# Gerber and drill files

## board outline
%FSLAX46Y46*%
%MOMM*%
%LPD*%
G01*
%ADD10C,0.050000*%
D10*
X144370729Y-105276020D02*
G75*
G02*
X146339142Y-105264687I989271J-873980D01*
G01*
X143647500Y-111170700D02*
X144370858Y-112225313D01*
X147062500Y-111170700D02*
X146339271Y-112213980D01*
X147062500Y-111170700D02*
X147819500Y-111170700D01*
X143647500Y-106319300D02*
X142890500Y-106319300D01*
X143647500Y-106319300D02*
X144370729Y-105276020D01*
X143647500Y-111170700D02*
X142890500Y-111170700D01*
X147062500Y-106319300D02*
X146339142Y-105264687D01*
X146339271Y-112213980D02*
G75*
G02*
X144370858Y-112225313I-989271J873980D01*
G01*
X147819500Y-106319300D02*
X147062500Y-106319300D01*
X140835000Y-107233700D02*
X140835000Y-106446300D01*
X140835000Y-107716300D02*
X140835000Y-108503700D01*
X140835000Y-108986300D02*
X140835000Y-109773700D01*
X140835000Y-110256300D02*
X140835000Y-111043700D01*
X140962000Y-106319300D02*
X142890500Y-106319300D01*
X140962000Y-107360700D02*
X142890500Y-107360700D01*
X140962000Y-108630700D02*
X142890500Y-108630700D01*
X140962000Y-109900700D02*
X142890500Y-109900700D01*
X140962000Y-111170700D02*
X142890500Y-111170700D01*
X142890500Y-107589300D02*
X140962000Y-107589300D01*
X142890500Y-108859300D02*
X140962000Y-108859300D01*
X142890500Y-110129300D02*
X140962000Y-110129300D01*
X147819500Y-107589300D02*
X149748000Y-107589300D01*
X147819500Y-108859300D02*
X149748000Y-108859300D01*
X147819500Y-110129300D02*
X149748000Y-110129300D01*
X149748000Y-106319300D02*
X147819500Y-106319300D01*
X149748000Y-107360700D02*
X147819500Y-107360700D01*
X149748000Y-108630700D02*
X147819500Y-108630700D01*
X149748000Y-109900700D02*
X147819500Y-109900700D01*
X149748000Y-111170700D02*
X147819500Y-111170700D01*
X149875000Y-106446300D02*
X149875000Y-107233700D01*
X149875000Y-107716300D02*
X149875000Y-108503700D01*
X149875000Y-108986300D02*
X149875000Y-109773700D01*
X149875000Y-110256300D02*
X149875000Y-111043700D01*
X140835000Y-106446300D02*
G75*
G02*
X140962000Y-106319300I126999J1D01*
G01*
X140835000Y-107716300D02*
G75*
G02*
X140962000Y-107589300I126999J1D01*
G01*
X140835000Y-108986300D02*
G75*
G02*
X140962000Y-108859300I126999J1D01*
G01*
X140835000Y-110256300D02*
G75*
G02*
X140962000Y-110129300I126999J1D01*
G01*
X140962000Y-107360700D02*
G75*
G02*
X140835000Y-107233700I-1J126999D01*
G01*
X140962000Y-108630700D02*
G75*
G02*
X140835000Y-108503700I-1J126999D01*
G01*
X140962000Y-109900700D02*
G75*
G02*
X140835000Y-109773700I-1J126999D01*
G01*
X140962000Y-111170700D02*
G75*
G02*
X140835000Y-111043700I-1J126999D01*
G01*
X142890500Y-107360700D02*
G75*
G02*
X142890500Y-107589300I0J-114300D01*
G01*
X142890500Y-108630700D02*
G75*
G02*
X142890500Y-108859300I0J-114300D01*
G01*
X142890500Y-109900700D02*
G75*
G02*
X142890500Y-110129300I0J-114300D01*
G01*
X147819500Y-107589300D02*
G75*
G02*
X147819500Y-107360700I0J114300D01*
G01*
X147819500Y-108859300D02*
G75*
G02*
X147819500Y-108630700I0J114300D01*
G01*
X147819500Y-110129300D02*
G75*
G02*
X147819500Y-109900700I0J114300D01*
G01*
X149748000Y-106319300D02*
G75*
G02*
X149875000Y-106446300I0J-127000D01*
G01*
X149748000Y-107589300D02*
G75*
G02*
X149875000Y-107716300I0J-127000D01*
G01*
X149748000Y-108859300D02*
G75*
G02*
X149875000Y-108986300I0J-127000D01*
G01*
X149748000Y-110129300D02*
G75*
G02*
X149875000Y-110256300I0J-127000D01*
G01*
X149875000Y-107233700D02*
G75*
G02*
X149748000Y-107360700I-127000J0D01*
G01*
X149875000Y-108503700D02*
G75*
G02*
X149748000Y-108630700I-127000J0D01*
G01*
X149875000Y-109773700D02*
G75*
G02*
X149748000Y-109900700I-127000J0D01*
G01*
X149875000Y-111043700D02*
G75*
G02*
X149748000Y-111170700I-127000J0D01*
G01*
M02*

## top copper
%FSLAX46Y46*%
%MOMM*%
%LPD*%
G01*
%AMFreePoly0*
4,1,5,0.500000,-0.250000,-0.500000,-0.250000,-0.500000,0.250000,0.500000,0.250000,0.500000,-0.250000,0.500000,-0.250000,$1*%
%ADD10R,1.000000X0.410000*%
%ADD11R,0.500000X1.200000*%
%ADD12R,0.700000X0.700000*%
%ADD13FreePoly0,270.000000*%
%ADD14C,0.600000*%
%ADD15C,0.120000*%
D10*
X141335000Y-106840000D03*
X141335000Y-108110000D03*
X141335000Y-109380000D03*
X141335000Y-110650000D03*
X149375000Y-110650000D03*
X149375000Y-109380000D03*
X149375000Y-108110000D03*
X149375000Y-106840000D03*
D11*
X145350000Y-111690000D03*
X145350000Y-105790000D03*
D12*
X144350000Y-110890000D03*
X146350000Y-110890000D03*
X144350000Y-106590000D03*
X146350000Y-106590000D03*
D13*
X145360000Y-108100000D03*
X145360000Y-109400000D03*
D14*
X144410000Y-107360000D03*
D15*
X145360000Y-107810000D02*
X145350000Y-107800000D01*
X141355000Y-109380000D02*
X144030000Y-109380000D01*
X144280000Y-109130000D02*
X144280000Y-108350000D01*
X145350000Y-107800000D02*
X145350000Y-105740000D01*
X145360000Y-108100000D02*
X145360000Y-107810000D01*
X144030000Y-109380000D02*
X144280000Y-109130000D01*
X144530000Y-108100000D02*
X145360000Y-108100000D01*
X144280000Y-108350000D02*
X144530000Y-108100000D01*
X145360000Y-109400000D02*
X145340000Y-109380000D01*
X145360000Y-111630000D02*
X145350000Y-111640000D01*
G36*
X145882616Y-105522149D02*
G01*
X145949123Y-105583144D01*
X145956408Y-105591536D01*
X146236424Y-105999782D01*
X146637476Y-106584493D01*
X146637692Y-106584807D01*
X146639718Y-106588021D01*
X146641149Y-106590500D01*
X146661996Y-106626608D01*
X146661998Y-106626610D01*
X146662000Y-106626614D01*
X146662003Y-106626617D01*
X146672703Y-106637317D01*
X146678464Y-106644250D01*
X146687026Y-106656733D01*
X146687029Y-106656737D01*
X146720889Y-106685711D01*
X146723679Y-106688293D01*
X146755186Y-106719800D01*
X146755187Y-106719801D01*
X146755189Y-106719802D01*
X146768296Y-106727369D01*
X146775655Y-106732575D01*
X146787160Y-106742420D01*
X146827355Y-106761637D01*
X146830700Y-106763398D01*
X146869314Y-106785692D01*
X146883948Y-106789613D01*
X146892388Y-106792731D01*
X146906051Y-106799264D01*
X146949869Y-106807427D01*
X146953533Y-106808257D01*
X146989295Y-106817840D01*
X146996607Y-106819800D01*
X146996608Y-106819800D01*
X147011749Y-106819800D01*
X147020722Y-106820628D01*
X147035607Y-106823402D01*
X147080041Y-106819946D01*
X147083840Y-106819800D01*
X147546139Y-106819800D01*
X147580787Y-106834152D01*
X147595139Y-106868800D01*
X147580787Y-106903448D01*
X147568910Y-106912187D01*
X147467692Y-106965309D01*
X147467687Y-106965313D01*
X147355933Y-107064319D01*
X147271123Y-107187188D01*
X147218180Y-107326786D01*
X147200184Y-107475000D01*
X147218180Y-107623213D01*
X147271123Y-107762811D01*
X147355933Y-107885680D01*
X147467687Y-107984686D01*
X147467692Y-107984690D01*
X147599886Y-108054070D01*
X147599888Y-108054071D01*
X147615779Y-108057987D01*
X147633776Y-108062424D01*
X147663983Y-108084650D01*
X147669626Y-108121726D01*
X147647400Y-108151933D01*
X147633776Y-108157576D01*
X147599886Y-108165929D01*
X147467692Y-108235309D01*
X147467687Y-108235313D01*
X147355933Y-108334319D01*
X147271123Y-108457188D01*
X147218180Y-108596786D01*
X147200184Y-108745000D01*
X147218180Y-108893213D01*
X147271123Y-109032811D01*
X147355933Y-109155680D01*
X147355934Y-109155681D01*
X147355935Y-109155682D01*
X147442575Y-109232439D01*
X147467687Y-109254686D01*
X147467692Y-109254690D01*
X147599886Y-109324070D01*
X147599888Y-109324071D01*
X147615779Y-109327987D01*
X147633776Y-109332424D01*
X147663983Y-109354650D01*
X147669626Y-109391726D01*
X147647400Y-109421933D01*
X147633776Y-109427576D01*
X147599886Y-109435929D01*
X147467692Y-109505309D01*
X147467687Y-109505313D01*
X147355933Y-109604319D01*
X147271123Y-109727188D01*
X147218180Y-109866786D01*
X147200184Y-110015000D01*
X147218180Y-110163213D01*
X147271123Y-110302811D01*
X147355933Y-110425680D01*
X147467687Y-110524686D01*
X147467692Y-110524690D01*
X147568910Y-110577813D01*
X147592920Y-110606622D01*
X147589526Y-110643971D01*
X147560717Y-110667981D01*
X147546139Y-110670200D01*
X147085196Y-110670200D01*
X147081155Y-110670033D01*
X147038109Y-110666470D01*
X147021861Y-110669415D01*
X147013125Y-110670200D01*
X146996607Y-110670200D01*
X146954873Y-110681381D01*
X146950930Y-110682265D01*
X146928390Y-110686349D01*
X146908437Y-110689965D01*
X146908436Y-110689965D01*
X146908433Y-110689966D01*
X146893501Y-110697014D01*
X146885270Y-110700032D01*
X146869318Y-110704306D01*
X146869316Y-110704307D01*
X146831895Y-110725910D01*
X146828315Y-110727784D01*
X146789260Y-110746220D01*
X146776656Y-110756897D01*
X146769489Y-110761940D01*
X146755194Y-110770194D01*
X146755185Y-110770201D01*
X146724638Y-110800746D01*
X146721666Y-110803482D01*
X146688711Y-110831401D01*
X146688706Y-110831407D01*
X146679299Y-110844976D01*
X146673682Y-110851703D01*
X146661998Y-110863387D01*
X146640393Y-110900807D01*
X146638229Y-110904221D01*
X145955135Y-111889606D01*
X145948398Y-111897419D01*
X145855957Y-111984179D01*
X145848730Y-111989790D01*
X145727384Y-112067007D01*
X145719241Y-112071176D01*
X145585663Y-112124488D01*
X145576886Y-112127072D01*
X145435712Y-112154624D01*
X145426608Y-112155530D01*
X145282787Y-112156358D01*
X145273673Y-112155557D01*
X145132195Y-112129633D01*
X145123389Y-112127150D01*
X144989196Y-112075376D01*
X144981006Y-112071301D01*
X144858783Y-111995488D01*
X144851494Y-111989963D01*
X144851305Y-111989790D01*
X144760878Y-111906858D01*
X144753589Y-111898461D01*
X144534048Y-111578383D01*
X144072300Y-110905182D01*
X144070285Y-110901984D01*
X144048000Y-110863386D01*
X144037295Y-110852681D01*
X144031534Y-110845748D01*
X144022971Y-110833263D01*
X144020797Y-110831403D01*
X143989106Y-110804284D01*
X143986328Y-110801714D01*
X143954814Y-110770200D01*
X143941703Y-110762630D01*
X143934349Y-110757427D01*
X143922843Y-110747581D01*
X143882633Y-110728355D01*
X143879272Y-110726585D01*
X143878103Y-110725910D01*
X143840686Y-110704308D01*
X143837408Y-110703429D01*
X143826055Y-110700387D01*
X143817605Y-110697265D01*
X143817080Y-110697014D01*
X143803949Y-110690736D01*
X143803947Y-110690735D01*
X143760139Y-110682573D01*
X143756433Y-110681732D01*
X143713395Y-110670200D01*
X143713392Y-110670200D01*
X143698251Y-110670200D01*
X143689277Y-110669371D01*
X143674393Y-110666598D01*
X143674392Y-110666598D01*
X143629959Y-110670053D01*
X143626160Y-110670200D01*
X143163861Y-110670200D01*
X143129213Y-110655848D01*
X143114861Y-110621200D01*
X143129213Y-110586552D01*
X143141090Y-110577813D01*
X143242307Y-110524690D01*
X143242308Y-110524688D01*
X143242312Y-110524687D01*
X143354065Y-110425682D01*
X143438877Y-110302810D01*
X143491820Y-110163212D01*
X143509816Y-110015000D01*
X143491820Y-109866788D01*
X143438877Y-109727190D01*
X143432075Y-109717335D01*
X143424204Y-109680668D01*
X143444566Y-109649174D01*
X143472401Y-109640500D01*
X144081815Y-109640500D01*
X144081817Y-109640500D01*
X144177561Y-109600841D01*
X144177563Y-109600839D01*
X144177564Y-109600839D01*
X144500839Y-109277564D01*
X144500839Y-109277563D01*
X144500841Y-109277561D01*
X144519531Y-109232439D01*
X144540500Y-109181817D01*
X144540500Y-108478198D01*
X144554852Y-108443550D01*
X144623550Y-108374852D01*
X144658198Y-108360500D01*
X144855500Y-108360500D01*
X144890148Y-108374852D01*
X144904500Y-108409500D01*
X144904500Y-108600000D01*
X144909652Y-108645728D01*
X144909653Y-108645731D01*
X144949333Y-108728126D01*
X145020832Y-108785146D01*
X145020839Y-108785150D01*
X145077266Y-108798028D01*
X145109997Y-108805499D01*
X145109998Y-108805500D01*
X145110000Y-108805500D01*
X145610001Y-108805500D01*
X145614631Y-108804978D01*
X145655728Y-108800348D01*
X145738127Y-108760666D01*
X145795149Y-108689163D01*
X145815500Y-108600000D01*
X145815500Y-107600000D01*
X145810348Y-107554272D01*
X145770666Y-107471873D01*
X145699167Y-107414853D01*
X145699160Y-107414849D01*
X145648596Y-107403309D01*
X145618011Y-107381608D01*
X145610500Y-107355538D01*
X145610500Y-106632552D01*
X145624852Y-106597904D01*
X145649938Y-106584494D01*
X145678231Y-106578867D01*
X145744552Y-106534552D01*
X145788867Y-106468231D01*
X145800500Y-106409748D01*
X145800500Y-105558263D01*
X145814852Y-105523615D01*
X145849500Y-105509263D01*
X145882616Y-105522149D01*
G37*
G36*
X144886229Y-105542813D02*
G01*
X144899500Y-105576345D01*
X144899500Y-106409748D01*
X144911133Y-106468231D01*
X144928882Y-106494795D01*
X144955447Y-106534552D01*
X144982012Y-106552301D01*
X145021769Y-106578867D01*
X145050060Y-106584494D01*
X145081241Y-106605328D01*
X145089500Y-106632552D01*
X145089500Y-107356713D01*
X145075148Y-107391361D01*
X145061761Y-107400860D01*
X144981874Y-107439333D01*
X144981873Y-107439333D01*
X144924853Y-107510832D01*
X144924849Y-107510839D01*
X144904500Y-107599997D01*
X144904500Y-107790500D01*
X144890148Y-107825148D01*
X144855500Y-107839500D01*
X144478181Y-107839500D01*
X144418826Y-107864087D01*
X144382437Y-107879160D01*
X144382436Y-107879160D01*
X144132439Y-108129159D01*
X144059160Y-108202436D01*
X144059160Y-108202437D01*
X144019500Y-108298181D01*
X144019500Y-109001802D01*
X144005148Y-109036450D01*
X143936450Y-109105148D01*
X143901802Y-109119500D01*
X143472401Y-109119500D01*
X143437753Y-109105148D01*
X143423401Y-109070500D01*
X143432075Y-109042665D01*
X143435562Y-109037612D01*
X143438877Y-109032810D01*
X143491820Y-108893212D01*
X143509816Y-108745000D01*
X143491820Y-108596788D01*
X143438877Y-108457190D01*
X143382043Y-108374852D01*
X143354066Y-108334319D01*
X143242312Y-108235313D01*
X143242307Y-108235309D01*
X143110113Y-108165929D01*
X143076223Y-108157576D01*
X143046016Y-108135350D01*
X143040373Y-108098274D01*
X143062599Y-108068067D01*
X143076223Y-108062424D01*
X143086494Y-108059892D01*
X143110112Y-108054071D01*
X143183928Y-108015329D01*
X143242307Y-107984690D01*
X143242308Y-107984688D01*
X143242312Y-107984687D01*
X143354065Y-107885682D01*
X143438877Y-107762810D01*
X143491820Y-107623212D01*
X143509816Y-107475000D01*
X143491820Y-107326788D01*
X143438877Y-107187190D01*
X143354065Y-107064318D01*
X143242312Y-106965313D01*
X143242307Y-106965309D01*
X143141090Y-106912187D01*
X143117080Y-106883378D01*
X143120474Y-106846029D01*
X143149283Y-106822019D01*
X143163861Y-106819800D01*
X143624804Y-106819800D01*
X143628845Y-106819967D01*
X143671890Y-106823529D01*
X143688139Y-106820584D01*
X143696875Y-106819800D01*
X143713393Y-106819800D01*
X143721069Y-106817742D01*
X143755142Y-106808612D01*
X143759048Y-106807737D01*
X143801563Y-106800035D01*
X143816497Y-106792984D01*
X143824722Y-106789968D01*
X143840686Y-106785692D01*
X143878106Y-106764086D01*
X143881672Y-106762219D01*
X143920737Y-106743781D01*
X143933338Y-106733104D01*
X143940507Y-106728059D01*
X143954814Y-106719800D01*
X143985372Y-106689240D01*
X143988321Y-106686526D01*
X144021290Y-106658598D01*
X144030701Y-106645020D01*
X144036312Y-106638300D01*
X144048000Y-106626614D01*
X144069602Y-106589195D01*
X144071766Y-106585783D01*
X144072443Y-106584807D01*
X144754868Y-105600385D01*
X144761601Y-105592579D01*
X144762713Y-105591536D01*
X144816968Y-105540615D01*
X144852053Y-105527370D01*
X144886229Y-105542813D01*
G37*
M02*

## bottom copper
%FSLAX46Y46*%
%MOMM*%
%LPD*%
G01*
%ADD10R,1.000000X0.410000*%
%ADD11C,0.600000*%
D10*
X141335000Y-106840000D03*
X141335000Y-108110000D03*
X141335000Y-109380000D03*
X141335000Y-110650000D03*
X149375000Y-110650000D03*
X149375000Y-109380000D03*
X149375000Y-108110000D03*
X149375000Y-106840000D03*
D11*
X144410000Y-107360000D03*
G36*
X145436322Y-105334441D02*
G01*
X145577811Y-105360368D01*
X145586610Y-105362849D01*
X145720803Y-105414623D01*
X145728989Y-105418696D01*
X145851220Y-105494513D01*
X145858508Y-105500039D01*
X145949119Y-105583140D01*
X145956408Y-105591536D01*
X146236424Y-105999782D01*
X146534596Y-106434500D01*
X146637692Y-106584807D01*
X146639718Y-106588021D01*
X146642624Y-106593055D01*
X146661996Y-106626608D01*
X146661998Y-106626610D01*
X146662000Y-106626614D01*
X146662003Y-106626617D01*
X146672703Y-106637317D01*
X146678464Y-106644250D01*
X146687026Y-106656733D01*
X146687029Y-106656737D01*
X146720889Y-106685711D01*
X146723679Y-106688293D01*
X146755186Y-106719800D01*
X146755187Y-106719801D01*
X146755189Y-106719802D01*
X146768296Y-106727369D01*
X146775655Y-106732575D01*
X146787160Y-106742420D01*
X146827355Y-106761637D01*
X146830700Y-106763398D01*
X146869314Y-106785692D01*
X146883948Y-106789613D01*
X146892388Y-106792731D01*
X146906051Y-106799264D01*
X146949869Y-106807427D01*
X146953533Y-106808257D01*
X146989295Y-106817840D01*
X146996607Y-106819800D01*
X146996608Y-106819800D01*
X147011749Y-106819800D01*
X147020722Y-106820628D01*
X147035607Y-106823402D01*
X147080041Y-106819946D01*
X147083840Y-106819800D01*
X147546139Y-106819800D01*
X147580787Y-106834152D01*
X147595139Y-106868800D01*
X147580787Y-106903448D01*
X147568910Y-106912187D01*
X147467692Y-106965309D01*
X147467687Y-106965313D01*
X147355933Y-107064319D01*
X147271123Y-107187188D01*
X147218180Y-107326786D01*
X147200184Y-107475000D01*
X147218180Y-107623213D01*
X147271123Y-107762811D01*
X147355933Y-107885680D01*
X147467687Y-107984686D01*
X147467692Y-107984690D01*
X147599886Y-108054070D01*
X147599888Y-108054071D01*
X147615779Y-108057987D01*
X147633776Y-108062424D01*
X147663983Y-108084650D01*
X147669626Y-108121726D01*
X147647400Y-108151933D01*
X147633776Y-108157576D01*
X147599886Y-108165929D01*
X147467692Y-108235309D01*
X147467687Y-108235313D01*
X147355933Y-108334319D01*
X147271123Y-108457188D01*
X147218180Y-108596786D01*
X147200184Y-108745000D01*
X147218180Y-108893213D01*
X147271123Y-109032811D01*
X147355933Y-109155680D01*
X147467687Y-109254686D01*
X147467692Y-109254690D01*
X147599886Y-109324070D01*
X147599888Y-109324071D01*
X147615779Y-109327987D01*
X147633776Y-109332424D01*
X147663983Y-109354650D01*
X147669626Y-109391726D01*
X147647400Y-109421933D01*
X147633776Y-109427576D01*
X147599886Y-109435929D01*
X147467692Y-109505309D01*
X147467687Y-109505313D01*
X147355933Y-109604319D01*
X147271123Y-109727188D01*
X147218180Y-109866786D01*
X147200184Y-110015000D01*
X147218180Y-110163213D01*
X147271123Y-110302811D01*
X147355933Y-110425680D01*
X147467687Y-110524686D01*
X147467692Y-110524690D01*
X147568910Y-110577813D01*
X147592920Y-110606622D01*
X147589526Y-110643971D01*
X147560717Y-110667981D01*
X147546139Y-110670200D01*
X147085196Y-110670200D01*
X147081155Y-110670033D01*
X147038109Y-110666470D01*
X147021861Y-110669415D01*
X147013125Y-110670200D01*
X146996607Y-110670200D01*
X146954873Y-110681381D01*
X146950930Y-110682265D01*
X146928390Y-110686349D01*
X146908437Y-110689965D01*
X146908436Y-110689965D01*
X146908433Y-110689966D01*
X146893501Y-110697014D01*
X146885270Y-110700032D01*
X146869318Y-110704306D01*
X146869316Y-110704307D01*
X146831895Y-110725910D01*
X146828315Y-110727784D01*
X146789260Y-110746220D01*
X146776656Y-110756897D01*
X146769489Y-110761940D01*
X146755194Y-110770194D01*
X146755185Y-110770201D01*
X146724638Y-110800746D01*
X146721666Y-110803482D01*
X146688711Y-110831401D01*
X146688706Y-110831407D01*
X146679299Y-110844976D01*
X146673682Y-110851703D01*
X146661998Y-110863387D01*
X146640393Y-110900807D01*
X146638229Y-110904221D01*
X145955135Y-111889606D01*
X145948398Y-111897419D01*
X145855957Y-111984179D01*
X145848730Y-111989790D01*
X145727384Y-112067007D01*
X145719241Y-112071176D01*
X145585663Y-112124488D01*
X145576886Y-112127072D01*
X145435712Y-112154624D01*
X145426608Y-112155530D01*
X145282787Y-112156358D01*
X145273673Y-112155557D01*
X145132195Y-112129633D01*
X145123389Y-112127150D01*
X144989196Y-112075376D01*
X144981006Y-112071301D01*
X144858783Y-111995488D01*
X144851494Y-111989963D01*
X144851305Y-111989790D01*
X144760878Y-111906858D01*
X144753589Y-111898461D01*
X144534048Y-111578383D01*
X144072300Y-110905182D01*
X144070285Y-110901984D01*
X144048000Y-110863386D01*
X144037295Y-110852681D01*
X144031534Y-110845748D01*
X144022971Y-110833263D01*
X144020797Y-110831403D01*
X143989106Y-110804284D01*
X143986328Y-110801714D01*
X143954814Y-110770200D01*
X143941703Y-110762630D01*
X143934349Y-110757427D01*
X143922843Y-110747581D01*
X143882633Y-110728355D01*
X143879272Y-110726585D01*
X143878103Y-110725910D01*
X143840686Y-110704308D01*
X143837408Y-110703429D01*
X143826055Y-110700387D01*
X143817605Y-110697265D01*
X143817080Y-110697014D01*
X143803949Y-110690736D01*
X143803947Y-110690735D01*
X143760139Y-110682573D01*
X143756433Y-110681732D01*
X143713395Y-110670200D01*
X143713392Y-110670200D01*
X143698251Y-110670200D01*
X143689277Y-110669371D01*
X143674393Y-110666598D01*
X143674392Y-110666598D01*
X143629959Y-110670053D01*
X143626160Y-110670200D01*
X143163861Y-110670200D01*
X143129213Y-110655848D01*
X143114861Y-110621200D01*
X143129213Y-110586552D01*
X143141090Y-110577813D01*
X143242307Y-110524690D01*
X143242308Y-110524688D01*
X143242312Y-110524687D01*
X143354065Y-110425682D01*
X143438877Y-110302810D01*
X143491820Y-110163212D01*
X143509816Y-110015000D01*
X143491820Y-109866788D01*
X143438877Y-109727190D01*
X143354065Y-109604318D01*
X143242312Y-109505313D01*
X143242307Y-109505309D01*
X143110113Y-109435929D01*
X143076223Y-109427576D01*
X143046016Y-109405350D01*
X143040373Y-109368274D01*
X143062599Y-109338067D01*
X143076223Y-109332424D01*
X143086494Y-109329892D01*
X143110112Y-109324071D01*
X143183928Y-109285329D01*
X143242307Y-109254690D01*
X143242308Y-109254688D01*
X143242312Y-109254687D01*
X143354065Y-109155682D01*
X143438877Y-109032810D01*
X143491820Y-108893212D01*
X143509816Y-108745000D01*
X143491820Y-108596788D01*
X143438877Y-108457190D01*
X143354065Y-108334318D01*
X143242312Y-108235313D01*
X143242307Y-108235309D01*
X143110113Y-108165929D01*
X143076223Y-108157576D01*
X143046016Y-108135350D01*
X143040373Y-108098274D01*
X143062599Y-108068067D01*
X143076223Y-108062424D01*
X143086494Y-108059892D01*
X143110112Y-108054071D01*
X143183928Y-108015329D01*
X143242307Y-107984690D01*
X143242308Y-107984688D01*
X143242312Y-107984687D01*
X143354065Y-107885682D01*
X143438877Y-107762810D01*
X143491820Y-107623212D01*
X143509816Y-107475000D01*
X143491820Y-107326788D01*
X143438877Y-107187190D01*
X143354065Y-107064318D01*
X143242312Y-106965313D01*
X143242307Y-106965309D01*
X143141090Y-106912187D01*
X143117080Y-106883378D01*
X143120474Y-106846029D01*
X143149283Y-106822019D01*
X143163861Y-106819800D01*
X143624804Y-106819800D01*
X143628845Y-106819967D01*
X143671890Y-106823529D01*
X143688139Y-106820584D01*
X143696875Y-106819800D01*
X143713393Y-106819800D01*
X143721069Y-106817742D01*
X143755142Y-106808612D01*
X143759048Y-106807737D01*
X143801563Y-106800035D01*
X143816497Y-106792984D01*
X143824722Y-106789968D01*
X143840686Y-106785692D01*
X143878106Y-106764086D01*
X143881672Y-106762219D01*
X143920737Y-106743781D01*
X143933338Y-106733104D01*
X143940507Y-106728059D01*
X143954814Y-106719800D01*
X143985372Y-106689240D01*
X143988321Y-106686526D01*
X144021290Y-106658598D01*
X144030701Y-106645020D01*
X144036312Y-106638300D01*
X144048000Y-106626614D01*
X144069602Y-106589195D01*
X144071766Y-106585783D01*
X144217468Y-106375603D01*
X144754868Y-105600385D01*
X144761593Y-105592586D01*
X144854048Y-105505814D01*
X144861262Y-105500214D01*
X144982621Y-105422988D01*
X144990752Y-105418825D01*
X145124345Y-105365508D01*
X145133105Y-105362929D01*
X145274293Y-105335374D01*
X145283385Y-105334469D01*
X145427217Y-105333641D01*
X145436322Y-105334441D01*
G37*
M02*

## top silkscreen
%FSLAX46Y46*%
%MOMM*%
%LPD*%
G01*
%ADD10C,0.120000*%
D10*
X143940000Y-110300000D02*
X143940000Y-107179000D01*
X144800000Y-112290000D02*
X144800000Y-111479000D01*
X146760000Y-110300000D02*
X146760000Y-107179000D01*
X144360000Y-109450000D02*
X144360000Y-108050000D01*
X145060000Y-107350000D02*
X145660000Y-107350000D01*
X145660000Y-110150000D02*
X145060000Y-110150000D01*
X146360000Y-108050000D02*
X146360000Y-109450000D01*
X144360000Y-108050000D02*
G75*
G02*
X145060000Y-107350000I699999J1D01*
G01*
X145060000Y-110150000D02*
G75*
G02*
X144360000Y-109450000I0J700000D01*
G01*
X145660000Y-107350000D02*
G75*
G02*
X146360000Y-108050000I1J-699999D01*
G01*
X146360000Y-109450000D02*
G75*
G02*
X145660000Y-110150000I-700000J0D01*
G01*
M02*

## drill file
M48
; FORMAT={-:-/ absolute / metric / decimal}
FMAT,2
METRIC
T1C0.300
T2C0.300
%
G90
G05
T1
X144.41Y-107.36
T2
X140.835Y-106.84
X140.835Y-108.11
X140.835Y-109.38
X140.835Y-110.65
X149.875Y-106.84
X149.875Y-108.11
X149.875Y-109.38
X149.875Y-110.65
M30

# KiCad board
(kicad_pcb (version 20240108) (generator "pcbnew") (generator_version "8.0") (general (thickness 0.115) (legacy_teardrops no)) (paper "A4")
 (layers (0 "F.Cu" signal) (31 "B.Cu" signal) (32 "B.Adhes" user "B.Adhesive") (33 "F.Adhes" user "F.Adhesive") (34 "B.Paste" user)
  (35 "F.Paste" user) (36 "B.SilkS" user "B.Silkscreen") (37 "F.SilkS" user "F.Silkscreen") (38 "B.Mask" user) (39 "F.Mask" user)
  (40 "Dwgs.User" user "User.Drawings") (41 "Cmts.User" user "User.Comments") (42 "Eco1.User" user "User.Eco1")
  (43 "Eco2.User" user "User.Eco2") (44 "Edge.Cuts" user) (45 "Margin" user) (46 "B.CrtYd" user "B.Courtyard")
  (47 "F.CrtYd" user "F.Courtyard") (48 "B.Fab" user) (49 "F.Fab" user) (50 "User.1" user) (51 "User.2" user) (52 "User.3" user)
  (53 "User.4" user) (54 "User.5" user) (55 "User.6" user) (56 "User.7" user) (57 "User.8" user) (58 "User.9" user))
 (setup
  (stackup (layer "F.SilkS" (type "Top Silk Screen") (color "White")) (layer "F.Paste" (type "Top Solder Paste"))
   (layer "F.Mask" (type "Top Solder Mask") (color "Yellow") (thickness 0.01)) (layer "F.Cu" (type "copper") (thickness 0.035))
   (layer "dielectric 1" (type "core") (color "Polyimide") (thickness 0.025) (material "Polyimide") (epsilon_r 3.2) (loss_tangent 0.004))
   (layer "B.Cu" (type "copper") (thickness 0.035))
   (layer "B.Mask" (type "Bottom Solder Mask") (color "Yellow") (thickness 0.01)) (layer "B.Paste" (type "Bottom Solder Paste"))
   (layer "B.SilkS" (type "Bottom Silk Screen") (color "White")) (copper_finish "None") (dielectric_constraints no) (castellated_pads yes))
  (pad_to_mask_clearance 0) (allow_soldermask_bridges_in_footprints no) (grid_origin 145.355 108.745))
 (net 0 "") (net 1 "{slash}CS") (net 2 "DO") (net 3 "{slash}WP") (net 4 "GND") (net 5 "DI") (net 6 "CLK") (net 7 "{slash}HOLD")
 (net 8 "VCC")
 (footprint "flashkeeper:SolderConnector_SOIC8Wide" (layer "F.Cu") (at 145.355 108.745)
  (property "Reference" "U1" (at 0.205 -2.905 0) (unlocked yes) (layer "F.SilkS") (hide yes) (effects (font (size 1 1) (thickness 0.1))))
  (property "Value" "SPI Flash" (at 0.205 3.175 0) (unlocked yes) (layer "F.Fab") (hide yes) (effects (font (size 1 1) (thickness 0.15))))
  (fp_line (start -4.52 -1.5113) (end -4.52 -2.2987) (stroke (width 0.05) (type default)) (layer "Edge.Cuts"))
  (fp_line (start -4.52 -1.0287) (end -4.52 -0.2413) (stroke (width 0.05) (type default)) (layer "Edge.Cuts"))
  (fp_line (start -4.52 0.2413) (end -4.52 1.0287) (stroke (width 0.05) (type default)) (layer "Edge.Cuts"))
  (fp_line (start -4.52 1.5113) (end -4.52 2.2987) (stroke (width 0.05) (type default)) (layer "Edge.Cuts"))
  (fp_line (start -4.393 -2.4257) (end -2.4645 -2.4257) (stroke (width 0.05) (type default)) (layer "Edge.Cuts"))
  (fp_line (start -4.393 -1.3843) (end -2.4645 -1.3843) (stroke (width 0.05) (type default)) (layer "Edge.Cuts"))
  (fp_line (start -4.393 -0.1143) (end -2.4645 -0.1143) (stroke (width 0.05) (type default)) (layer "Edge.Cuts"))
  (fp_line (start -4.393 1.1557) (end -2.4645 1.1557) (stroke (width 0.05) (type default)) (layer "Edge.Cuts"))
  (fp_line (start -4.393 2.4257) (end -2.4645 2.4257) (stroke (width 0.05) (type default)) (layer "Edge.Cuts"))
  (fp_line (start -2.4645 -1.1557) (end -4.393 -1.1557) (stroke (width 0.05) (type default)) (layer "Edge.Cuts"))
  (fp_line (start -2.4645 0.1143) (end -4.393 0.1143) (stroke (width 0.05) (type default)) (layer "Edge.Cuts"))
  (fp_line (start -2.4645 1.3843) (end -4.393 1.3843) (stroke (width 0.05) (type default)) (layer "Edge.Cuts"))
  (fp_line (start 2.4645 -1.1557) (end 4.393 -1.1557) (stroke (width 0.05) (type default)) (layer "Edge.Cuts"))
  (fp_line (start 2.4645 0.1143) (end 4.393 0.1143) (stroke (width 0.05) (type default)) (layer "Edge.Cuts"))
  (fp_line (start 2.4645 1.3843) (end 4.393 1.3843) (stroke (width 0.05) (type default)) (layer "Edge.Cuts"))
  (fp_line (start 4.393 -2.4257) (end 2.4645 -2.4257) (stroke (width 0.05) (type default)) (layer "Edge.Cuts"))
  (fp_line (start 4.393 -1.3843) (end 2.4645 -1.3843) (stroke (width 0.05) (type default)) (layer "Edge.Cuts"))
  (fp_line (start 4.393 -0.1143) (end 2.4645 -0.1143) (stroke (width 0.05) (type default)) (layer "Edge.Cuts"))
  (fp_line (start 4.393 1.1557) (end 2.4645 1.1557) (stroke (width 0.05) (type default)) (layer "Edge.Cuts"))
  (fp_line (start 4.393 2.4257) (end 2.4645 2.4257) (stroke (width 0.05) (type default)) (layer "Edge.Cuts"))
  (fp_line (start 4.52 -2.2987) (end 4.52 -1.5113) (stroke (width 0.05) (type default)) (layer "Edge.Cuts"))
  (fp_line (start 4.52 -1.0287) (end 4.52 -0.2413) (stroke (width 0.05) (type default)) (layer "Edge.Cuts"))
  (fp_line (start 4.52 0.2413) (end 4.52 1.0287) (stroke (width 0.05) (type default)) (layer "Edge.Cuts"))
  (fp_line (start 4.52 1.5113) (end 4.52 2.2987) (stroke (width 0.05) (type default)) (layer "Edge.Cuts"))
  (fp_arc (start -4.52 -2.2987) (mid -4.482803 -2.388503) (end -4.393 -2.4257) (stroke (width 0.05) (type default)) (layer "Edge.Cuts"))
  (fp_arc (start -4.52 -1.0287) (mid -4.482803 -1.118503) (end -4.393 -1.1557) (stroke (width 0.05) (type default)) (layer "Edge.Cuts"))
  (fp_arc (start -4.52 0.2413) (mid -4.482803 0.151497) (end -4.393 0.1143) (stroke (width 0.05) (type default)) (layer "Edge.Cuts"))
  (fp_arc (start -4.52 1.5113) (mid -4.482803 1.421497) (end -4.393 1.3843) (stroke (width 0.05) (type default)) (layer "Edge.Cuts"))
  (fp_arc (start -4.393 -1.3843) (mid -4.482803 -1.421497) (end -4.52 -1.5113) (stroke (width 0.05) (type default)) (layer "Edge.Cuts"))
  (fp_arc (start -4.393 -0.1143) (mid -4.482803 -0.151497) (end -4.52 -0.2413) (stroke (width 0.05) (type default)) (layer "Edge.Cuts"))
  (fp_arc (start -4.393 1.1557) (mid -4.482803 1.118503) (end -4.52 1.0287) (stroke (width 0.05) (type default)) (layer "Edge.Cuts"))
  (fp_arc (start -4.393 2.4257) (mid -4.482803 2.388503) (end -4.52 2.2987) (stroke (width 0.05) (type default)) (layer "Edge.Cuts"))
  (fp_arc (start -2.4645 -1.3843) (mid -2.3502 -1.27) (end -2.4645 -1.1557) (stroke (width 0.05) (type default)) (layer "Edge.Cuts"))
  (fp_arc (start -2.4645 -0.1143) (mid -2.3502 0) (end -2.4645 0.1143) (stroke (width 0.05) (type default)) (layer "Edge.Cuts"))
  (fp_arc (start -2.4645 1.1557) (mid -2.3502 1.27) (end -2.4645 1.3843) (stroke (width 0.05) (type default)) (layer "Edge.Cuts"))
  (fp_arc (start 2.4645 -1.1557) (mid 2.3502 -1.27) (end 2.4645 -1.3843) (stroke (width 0.05) (type default)) (layer "Edge.Cuts"))
  (fp_arc (start 2.4645 0.1143) (mid 2.3502 0) (end 2.4645 -0.1143) (stroke (width 0.05) (type default)) (layer "Edge.Cuts"))
  (fp_arc (start 2.4645 1.3843) (mid 2.3502 1.27) (end 2.4645 1.1557) (stroke (width 0.05) (type default)) (layer "Edge.Cuts"))
  (fp_arc (start 4.393 -2.4257) (mid 4.482803 -2.388503) (end 4.52 -2.2987) (stroke (width 0.05) (type default)) (layer "Edge.Cuts"))
  (fp_arc (start 4.393 -1.1557) (mid 4.482803 -1.118503) (end 4.52 -1.0287) (stroke (width 0.05) (type default)) (layer "Edge.Cuts"))
  (fp_arc (start 4.393 0.1143) (mid 4.482803 0.151497) (end 4.52 0.2413) (stroke (width 0.05) (type default)) (layer "Edge.Cuts"))
  (fp_arc (start 4.393 1.3843) (mid 4.482803 1.421497) (end 4.52 1.5113) (stroke (width 0.05) (type default)) (layer "Edge.Cuts"))
  (fp_arc (start 4.52 -1.5113) (mid 4.482803 -1.421497) (end 4.393 -1.3843) (stroke (width 0.05) (type default)) (layer "Edge.Cuts"))
  (fp_arc (start 4.52 -0.2413) (mid 4.482803 -0.151497) (end 4.393 -0.1143) (stroke (width 0.05) (type default)) (layer "Edge.Cuts"))
  (fp_arc (start 4.52 1.0287) (mid 4.482803 1.118503) (end 4.393 1.1557) (stroke (width 0.05) (type default)) (layer "Edge.Cuts"))
  (fp_arc (start 4.52 2.2987) (mid 4.482803 2.388503) (end 4.393 2.4257) (stroke (width 0.05) (type default)) (layer "Edge.Cuts"))
  (pad "1" thru_hole rect (at -4.52 -1.905) (size 1 0.41) (drill 0.3 (offset 0.5 0)) (layers "*.Cu" "*.Mask") (remove_unused_layers no)
   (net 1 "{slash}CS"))
  (pad "2" thru_hole rect (at -4.52 -0.635) (size 1 0.41) (drill 0.3 (offset 0.5 0)) (layers "*.Cu" "*.Mask") (remove_unused_layers no)
   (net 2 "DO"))
  (pad "3" thru_hole rect (at -4.52 0.635) (size 1 0.41) (drill 0.3 (offset 0.5 0)) (layers "*.Cu" "*.Mask") (remove_unused_layers no)
   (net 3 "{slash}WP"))
  (pad "4" thru_hole rect (at -4.52 1.905) (size 1 0.41) (drill 0.3 (offset 0.5 0)) (layers "*.Cu" "*.Mask") (remove_unused_layers no)
   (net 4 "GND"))
  (pad "5" thru_hole rect (at 4.52 1.905 180) (size 1 0.41) (drill 0.3 (offset 0.5 0)) (layers "*.Cu" "*.Mask") (remove_unused_layers no)
   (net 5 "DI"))
  (pad "6" thru_hole rect (at 4.52 0.635 180) (size 1 0.41) (drill 0.3 (offset 0.5 0)) (layers "*.Cu" "*.Mask") (remove_unused_layers no)
   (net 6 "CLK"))
  (pad "7" thru_hole rect (at 4.52 -0.635 180) (size 1 0.41) (drill 0.3 (offset 0.5 0)) (layers "*.Cu" "*.Mask") (remove_unused_layers no)
   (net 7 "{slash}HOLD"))
  (pad "8" thru_hole rect (at 4.52 -1.905 180) (size 1 0.41) (drill 0.3 (offset 0.5 0)) (layers "*.Cu" "*.Mask") (remove_unused_layers no)
   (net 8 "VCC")))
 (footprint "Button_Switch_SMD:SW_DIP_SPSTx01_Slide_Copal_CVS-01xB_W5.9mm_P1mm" (layer "F.Cu") (at 145.35 108.74 90)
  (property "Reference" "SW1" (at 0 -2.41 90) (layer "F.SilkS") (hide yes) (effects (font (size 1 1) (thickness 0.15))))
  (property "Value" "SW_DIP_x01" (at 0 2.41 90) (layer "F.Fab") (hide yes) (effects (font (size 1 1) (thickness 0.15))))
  (fp_line (start -1.56 -1.41) (end 1.561 -1.41) (stroke (width 0.12) (type solid)) (layer "F.SilkS"))
  (fp_line (start -3.55 -0.55) (end -2.739 -0.55) (stroke (width 0.12) (type solid)) (layer "F.SilkS"))
  (fp_line (start -1.56 1.41) (end 1.561 1.41) (stroke (width 0.12) (type solid)) (layer "F.SilkS"))
  (pad "1" smd rect (at -2.95 0 90) (size 1.2 0.5) (layers "F.Cu" "F.Paste" "F.Mask") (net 4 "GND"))
  (pad "2" smd rect (at 2.95 0 90) (size 1.2 0.5) (layers "F.Cu" "F.Paste" "F.Mask") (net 3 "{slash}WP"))
  (pad "3" smd rect (at -2.15 -1 90) (size 0.7 0.7) (layers "F.Cu" "F.Paste" "F.Mask") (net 4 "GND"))
  (pad "3" smd rect (at -2.15 1 90) (size 0.7 0.7) (layers "F.Cu" "F.Paste" "F.Mask") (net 4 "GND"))
  (pad "3" smd rect (at 2.15 -1 90) (size 0.7 0.7) (layers "F.Cu" "F.Paste" "F.Mask") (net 4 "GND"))
  (pad "3" smd rect (at 2.15 1 90) (size 0.7 0.7) (layers "F.Cu" "F.Paste" "F.Mask") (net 4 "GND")))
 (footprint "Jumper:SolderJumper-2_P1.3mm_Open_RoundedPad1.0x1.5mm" (layer "F.Cu") (at 145.36 108.75 -90)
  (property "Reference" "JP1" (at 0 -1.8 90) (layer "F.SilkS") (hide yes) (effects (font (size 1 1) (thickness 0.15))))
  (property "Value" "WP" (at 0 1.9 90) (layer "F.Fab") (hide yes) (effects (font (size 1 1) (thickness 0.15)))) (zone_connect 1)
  (fp_line (start 0.7 1) (end -0.7 1) (stroke (width 0.12) (type solid)) (layer "F.SilkS"))
  (fp_line (start -1.4 0.3) (end -1.4 -0.3) (stroke (width 0.12) (type solid)) (layer "F.SilkS"))
  (fp_line (start 1.4 -0.3) (end 1.4 0.3) (stroke (width 0.12) (type solid)) (layer "F.SilkS"))
  (fp_line (start -0.7 -1) (end 0.7 -1) (stroke (width 0.12) (type solid)) (layer "F.SilkS"))
  (fp_arc (start -0.7 1) (mid -1.194975 0.794975) (end -1.4 0.3) (stroke (width 0.12) (type solid)) (layer "F.SilkS"))
  (fp_arc (start 1.4 0.3) (mid 1.194975 0.794975) (end 0.7 1) (stroke (width 0.12) (type solid)) (layer "F.SilkS"))
  (fp_arc (start -1.4 -0.3) (mid -1.194975 -0.794975) (end -0.7 -1) (stroke (width 0.12) (type solid)) (layer "F.SilkS"))
  (fp_arc (start 0.7 -1) (mid 1.194975 -0.794975) (end 1.4 -0.3) (stroke (width 0.12) (type solid)) (layer "F.SilkS"))
  (pad "1" smd custom (at -0.65 0 270) (size 1 0.5) (layers "F.Cu" "F.Mask") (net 3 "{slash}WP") (zone_connect 2) (thermal_bridge_angle 45)
   (options (clearance outline) (anchor rect)) (primitives))
  (pad "2" smd custom (at 0.65 0 270) (size 1 0.5) (layers "F.Cu" "F.Mask") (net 4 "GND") (zone_connect 2) (thermal_bridge_angle 45)
   (options (clearance outline) (anchor rect)) (primitives)))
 (gr_arc (start 144.370729 105.27602) (mid 145.3524 104.829985) (end 146.339142 105.264687) (stroke (width 0.05) (type default))
  (layer "Edge.Cuts"))
 (gr_line (start 143.6475 111.1707) (end 144.370858 112.225313) (stroke (width 0.05) (type default)) (layer "Edge.Cuts"))
 (gr_line (start 147.0625 111.1707) (end 146.339271 112.21398) (stroke (width 0.05) (type default)) (layer "Edge.Cuts"))
 (gr_line (start 147.0625 111.1707) (end 147.8195 111.1707) (stroke (width 0.05) (type default)) (layer "Edge.Cuts"))
 (gr_line (start 143.6475 106.3193) (end 142.8905 106.3193) (stroke (width 0.05) (type default)) (layer "Edge.Cuts"))
 (gr_line (start 143.6475 106.3193) (end 144.370729 105.27602) (stroke (width 0.05) (type default)) (layer "Edge.Cuts"))
 (gr_line (start 143.6475 111.1707) (end 142.8905 111.1707) (stroke (width 0.05) (type default)) (layer "Edge.Cuts"))
 (gr_line (start 147.0625 106.3193) (end 146.339142 105.264687) (stroke (width 0.05) (type default)) (layer "Edge.Cuts"))
 (gr_arc (start 146.339271 112.21398) (mid 145.3576 112.660015) (end 144.370858 112.225313) (stroke (width 0.05) (type default))
  (layer "Edge.Cuts"))
 (gr_line (start 147.8195 106.3193) (end 147.0625 106.3193) (stroke (width 0.05) (type default)) (layer "Edge.Cuts"))
 (segment (start 145.36 107.81) (end 145.35 107.8) (width 0.12) (layer "F.Cu") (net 3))
 (segment (start 141.355 109.38) (end 144.03 109.38) (width 0.12) (layer "F.Cu") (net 3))
 (segment (start 144.28 109.13) (end 144.28 108.35) (width 0.12) (layer "F.Cu") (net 3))
 (segment (start 145.35 107.8) (end 145.35 105.74) (width 0.12) (layer "F.Cu") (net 3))
 (segment (start 145.36 108.1) (end 145.36 107.81) (width 0.12) (layer "F.Cu") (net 3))
 (segment (start 144.03 109.38) (end 144.28 109.13) (width 0.12) (layer "F.Cu") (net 3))
 (segment (start 144.53 108.1) (end 145.36 108.1) (width 0.12) (layer "F.Cu") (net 3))
 (segment (start 144.28 108.35) (end 144.53 108.1) (width 0.12) (layer "F.Cu") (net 3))
 (segment (start 145.36 109.4) (end 145.34 109.38) (width 0.12) (layer "F.Cu") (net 4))
 (segment (start 145.36 111.63) (end 145.35 111.64) (width 0.12) (layer "F.Cu") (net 4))
 (via (at 144.41 107.36) (size 0.6) (drill 0.3) (layers "F.Cu" "B.Cu") (free yes) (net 4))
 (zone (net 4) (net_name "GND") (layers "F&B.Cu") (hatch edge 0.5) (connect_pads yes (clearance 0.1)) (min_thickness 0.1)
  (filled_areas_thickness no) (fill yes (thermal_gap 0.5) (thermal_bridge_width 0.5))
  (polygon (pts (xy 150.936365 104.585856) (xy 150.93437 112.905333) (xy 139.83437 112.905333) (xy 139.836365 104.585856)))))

